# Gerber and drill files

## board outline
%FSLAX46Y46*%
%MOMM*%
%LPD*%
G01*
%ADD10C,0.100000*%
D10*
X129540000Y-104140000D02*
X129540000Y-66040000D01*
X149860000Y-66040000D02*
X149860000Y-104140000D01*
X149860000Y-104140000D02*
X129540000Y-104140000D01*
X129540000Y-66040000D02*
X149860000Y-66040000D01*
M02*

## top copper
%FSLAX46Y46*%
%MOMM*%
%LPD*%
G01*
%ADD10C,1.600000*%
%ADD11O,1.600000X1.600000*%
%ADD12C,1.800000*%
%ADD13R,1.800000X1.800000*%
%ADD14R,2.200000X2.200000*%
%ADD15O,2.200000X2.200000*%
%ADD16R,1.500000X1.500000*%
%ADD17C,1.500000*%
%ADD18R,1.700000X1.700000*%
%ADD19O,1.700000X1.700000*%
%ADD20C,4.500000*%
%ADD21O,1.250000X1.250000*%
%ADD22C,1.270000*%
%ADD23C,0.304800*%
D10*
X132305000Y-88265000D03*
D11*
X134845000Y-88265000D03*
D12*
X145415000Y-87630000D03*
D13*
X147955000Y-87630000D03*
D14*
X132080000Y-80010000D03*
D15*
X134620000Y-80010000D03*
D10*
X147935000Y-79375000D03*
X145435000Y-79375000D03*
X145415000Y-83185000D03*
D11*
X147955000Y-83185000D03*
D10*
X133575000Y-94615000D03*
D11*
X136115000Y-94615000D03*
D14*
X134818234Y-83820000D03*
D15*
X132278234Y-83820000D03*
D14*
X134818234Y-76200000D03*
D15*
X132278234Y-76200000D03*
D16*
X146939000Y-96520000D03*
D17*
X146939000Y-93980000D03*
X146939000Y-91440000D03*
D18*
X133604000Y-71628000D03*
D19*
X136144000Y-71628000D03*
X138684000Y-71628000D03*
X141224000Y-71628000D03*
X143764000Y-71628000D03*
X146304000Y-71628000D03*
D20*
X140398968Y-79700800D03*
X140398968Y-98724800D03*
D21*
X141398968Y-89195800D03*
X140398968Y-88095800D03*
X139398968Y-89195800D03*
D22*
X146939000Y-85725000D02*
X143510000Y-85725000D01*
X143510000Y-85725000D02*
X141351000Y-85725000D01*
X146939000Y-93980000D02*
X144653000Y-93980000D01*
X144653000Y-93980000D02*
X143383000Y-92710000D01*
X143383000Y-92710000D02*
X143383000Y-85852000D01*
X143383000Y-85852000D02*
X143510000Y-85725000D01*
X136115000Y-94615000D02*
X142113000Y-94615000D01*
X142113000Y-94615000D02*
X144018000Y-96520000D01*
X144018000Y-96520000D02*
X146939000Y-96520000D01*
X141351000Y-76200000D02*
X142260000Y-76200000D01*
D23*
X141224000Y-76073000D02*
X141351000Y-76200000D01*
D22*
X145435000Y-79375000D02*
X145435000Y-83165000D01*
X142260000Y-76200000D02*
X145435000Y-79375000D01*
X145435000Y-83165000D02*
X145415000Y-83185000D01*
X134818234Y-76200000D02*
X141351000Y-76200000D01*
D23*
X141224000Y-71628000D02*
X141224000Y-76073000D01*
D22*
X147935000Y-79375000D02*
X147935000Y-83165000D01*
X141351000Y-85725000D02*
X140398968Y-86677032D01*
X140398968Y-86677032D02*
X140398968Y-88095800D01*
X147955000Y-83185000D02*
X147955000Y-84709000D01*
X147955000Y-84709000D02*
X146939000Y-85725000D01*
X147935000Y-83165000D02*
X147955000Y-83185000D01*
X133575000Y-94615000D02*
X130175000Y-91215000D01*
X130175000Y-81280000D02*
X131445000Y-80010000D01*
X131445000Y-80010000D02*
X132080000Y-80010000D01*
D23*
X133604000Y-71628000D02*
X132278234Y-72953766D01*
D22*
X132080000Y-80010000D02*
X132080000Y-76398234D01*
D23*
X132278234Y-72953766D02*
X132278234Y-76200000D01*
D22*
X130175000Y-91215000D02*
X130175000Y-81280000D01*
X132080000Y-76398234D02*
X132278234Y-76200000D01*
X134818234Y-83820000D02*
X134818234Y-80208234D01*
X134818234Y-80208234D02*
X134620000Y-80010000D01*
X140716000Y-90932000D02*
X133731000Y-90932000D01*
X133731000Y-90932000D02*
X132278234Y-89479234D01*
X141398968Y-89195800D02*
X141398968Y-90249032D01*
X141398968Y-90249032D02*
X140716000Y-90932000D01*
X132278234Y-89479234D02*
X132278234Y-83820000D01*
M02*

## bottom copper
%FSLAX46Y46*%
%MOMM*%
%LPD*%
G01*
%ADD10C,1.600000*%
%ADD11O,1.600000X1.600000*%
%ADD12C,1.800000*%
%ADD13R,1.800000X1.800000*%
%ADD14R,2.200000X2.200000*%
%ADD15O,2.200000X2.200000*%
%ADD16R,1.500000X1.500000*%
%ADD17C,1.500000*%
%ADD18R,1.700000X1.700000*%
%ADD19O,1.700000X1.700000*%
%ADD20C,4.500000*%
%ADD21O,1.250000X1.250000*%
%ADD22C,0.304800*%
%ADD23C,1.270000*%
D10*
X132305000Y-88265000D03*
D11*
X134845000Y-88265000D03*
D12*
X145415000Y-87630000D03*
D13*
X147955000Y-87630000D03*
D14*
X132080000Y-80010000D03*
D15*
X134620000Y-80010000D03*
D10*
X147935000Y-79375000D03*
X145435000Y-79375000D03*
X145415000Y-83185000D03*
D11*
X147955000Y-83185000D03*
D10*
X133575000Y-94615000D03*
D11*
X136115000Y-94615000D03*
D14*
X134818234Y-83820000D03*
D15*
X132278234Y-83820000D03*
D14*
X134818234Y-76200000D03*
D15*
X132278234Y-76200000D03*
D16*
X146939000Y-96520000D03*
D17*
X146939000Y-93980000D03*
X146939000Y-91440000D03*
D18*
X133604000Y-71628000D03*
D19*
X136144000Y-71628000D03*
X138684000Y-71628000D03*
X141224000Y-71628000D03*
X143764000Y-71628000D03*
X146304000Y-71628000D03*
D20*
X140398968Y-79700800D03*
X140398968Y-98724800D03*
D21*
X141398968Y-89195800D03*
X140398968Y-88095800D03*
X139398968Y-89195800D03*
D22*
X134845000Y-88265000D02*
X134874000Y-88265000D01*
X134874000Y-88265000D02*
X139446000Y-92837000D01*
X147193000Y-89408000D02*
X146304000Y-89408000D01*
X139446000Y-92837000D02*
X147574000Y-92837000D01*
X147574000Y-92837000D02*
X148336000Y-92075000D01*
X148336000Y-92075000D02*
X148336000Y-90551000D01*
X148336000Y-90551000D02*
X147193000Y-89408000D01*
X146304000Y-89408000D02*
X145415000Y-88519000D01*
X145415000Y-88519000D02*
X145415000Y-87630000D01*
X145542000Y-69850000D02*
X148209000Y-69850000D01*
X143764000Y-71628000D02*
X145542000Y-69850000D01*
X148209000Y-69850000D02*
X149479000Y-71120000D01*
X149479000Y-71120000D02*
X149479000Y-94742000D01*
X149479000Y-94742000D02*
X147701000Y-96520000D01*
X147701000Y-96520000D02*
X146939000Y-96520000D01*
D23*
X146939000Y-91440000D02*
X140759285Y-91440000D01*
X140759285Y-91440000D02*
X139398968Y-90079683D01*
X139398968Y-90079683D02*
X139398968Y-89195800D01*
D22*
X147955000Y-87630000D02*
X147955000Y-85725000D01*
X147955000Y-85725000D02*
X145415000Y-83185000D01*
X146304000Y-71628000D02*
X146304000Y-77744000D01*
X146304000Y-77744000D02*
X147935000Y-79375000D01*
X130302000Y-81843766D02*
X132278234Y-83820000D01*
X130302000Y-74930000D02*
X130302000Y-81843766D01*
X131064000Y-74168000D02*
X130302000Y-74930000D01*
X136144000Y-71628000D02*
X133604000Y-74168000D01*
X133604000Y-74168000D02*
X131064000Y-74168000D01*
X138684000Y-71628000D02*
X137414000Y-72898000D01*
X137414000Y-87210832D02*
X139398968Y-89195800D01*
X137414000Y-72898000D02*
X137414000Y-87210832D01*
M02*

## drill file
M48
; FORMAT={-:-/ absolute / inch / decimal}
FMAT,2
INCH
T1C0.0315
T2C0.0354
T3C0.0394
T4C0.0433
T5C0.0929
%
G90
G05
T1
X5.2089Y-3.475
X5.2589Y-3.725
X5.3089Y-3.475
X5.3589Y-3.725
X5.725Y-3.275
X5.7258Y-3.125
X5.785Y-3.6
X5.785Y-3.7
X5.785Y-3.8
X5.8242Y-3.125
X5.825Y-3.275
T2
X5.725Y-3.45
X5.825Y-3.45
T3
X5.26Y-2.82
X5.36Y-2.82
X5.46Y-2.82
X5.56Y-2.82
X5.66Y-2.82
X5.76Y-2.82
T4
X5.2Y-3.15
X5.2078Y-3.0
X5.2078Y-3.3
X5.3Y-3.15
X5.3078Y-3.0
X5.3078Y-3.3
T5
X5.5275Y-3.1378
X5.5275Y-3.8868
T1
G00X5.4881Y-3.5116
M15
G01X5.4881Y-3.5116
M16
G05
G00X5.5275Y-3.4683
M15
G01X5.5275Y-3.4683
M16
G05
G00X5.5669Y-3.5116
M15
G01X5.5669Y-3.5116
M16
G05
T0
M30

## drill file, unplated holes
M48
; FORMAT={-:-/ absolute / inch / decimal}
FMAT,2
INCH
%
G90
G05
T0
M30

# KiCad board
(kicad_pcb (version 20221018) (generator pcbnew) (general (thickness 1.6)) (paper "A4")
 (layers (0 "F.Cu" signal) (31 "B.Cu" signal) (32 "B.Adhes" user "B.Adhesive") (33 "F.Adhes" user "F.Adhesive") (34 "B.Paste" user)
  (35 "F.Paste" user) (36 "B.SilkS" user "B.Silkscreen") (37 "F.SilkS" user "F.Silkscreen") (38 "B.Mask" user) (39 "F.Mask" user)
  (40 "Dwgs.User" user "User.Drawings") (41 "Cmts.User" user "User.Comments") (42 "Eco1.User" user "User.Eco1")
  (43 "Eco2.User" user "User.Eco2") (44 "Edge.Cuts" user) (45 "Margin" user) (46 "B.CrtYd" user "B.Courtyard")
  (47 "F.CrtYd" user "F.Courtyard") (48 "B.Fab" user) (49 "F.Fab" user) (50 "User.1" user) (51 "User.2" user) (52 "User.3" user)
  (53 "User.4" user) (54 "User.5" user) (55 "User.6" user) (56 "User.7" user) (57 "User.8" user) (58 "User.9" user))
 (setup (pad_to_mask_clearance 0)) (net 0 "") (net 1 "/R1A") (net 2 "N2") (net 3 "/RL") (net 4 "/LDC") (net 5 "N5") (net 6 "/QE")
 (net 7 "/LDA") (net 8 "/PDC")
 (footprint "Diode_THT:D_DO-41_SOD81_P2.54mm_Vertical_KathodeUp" (layer "F.Cu") (at 132.08 80.01)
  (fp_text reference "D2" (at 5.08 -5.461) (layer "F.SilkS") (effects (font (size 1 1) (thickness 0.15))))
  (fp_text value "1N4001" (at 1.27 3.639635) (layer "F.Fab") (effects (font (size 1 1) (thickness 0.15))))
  (pad "1" thru_hole rect (at 0 0) (size 2.2 2.2) (drill 1.1) (layers "*.Cu" "*.Mask") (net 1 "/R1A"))
  (pad "2" thru_hole oval (at 2.54 0) (size 2.2 2.2) (drill 1.1) (layers "*.Cu" "*.Mask") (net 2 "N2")))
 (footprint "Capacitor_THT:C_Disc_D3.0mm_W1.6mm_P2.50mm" (layer "F.Cu") (at 145.435 79.375)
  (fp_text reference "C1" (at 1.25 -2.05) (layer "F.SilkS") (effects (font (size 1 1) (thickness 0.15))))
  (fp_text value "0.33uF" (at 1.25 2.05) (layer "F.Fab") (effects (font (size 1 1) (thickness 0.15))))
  (pad "1" thru_hole circle (at 0 0) (size 1.6 1.6) (drill 0.8) (layers "*.Cu" "*.Mask") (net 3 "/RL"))
  (pad "2" thru_hole circle (at 2.5 0) (size 1.6 1.6) (drill 0.8) (layers "*.Cu" "*.Mask") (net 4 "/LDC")))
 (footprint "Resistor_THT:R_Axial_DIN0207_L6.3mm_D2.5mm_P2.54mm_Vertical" (layer "F.Cu") (at 145.415 83.185)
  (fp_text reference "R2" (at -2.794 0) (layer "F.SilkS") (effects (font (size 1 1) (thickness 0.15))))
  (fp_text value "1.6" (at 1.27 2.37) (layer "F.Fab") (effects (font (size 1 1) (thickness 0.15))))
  (pad "1" thru_hole circle (at 0 0) (size 1.6 1.6) (drill 0.8) (layers "*.Cu" "*.Mask") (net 3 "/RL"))
  (pad "2" thru_hole oval (at 2.54 0) (size 1.6 1.6) (drill 0.8) (layers "*.Cu" "*.Mask") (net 4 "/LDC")))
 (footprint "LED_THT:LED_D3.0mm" (layer "F.Cu") (at 147.955 87.63 180)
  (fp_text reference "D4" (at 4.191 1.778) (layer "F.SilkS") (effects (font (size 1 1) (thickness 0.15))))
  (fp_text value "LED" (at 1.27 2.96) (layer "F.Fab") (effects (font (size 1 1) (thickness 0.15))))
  (pad "1" thru_hole rect (at 0 0 180) (size 1.8 1.8) (drill 0.9) (layers "*.Cu" "*.Mask") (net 3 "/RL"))
  (pad "2" thru_hole circle (at 2.54 0 180) (size 1.8 1.8) (drill 0.9) (layers "*.Cu" "*.Mask") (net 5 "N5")))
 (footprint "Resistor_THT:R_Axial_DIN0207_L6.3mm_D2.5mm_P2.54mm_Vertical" (layer "F.Cu") (at 133.575 94.615)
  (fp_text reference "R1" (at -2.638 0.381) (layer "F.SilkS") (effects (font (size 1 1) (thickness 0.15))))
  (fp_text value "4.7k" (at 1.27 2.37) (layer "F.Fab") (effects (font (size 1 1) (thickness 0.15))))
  (pad "1" thru_hole circle (at 0 0) (size 1.6 1.6) (drill 0.8) (layers "*.Cu" "*.Mask") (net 1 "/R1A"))
  (pad "2" thru_hole oval (at 2.54 0) (size 1.6 1.6) (drill 0.8) (layers "*.Cu" "*.Mask") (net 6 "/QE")))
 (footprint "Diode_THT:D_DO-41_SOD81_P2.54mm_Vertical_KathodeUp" (layer "F.Cu") (at 134.818234 83.82 180)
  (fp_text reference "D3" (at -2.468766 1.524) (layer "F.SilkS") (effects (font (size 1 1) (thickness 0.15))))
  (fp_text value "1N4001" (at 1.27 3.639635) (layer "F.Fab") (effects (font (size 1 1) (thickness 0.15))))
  (pad "1" thru_hole rect (at 0 0 180) (size 2.2 2.2) (drill 1.1) (layers "*.Cu" "*.Mask") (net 2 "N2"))
  (pad "2" thru_hole oval (at 2.54 0 180) (size 2.2 2.2) (drill 1.1) (layers "*.Cu" "*.Mask") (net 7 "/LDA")))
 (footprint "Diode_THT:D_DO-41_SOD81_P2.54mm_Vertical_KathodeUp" (layer "F.Cu") (at 134.818234 76.2 180)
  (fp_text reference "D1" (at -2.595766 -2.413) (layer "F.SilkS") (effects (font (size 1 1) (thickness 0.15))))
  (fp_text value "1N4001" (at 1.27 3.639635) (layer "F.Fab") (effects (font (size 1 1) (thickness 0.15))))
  (pad "1" thru_hole rect (at 0 0 180) (size 2.2 2.2) (drill 1.1) (layers "*.Cu" "*.Mask") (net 3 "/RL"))
  (pad "2" thru_hole oval (at 2.54 0 180) (size 2.2 2.2) (drill 1.1) (layers "*.Cu" "*.Mask") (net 1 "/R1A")))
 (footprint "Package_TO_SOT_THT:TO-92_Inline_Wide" (layer "F.Cu") (at 146.939 96.52 90)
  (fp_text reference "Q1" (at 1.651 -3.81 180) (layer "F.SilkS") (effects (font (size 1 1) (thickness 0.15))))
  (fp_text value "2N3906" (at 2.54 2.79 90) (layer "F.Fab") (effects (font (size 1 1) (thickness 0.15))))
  (pad "1" thru_hole rect (at 0 0 90) (size 1.5 1.5) (drill 0.8) (layers "*.Cu" "*.Mask") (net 6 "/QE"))
  (pad "2" thru_hole circle (at 2.54 0 90) (size 1.5 1.5) (drill 0.8) (layers "*.Cu" "*.Mask") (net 4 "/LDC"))
  (pad "3" thru_hole circle (at 5.08 0 90) (size 1.5 1.5) (drill 0.8) (layers "*.Cu" "*.Mask") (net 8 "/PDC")))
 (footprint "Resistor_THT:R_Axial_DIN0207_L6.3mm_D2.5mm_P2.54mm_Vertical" (layer "F.Cu") (at 132.305 88.265)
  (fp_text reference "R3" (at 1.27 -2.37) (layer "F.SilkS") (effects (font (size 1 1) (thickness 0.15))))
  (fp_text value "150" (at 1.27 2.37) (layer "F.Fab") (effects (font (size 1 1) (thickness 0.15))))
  (pad "1" thru_hole circle (at 0 0) (size 1.6 1.6) (drill 0.8) (layers "*.Cu" "*.Mask") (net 7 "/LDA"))
  (pad "2" thru_hole oval (at 2.54 0) (size 1.6 1.6) (drill 0.8) (layers "*.Cu" "*.Mask") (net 5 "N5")))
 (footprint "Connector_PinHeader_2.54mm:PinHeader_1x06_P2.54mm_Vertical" (layer "F.Cu") (at 133.604 71.628 90)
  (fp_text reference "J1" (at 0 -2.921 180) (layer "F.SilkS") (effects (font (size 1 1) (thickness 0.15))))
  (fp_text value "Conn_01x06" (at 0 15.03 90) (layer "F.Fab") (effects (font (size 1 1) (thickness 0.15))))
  (pad "1" thru_hole rect (at 0 0 90) (size 1.7 1.7) (drill 1) (layers "*.Cu" "*.Mask") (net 1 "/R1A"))
  (pad "2" thru_hole oval (at 0 2.54 90) (size 1.7 1.7) (drill 1) (layers "*.Cu" "*.Mask") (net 7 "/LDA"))
  (pad "3" thru_hole oval (at 0 5.08 90) (size 1.7 1.7) (drill 1) (layers "*.Cu" "*.Mask") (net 8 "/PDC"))
  (pad "4" thru_hole oval (at 0 7.62 90) (size 1.7 1.7) (drill 1) (layers "*.Cu" "*.Mask") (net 3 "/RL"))
  (pad "5" thru_hole oval (at 0 10.16 90) (size 1.7 1.7) (drill 1) (layers "*.Cu" "*.Mask") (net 6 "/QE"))
  (pad "6" thru_hole oval (at 0 12.7 90) (size 1.7 1.7) (drill 1) (layers "*.Cu" "*.Mask") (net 4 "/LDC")))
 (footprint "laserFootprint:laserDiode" (layer "B.Cu") (at 141.398968 89.1958 90)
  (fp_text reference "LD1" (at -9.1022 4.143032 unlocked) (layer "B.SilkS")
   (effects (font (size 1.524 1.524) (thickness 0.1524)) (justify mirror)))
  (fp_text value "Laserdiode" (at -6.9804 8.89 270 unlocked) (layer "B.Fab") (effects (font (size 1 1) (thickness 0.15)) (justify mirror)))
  (pad "1" thru_hole oval (at 0 -2) (size 1.25 1.25) (drill oval 0.8) (layers "*.Cu" "*.Mask") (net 8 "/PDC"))
  (pad "2" thru_hole oval (at 1.1 -1) (size 1.25 1.25) (drill oval 0.8) (layers "*.Cu" "*.Mask") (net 4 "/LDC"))
  (pad "3" thru_hole oval (at 0 0) (size 1.25 1.25) (drill oval 0.8) (layers "*.Cu" "*.Mask") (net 7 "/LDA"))
  (pad "4" thru_hole circle (at -9.529 -1 90) (size 4.5 4.5) (drill 2.36) (layers "*.Cu" "*.Mask"))
  (pad "4" thru_hole circle (at 9.495 -1 90) (size 4.5 4.5) (drill 2.36) (layers "*.Cu" "*.Mask")))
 (gr_line (start 129.54 104.14) (end 129.54 66.04) (stroke (width 0.1) (type default)) (layer "Edge.Cuts"))
 (gr_line (start 149.86 66.04) (end 149.86 104.14) (stroke (width 0.1) (type default)) (layer "Edge.Cuts"))
 (gr_line (start 149.86 104.14) (end 129.54 104.14) (stroke (width 0.1) (type default)) (layer "Edge.Cuts"))
 (gr_line (start 129.54 66.04) (end 149.86 66.04) (stroke (width 0.1) (type default)) (layer "Edge.Cuts"))
 (segment (start 141.351 76.2) (end 142.26 76.2) (width 1.27) (layer "F.Cu") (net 3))
 (segment (start 141.224 76.073) (end 141.351 76.2) (width 0.3048) (layer "F.Cu") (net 3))
 (segment (start 145.435 79.375) (end 145.435 83.165) (width 1.27) (layer "F.Cu") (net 3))
 (segment (start 142.26 76.2) (end 145.435 79.375) (width 1.27) (layer "F.Cu") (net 3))
 (segment (start 145.435 83.165) (end 145.415 83.185) (width 1.27) (layer "F.Cu") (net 3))
 (segment (start 134.818234 76.2) (end 141.351 76.2) (width 1.27) (layer "F.Cu") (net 3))
 (segment (start 141.224 71.628) (end 141.224 76.073) (width 0.3048) (layer "F.Cu") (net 3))
 (segment (start 147.955 87.63) (end 147.955 85.725) (width 0.3048) (layer "B.Cu") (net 3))
 (segment (start 147.955 85.725) (end 145.415 83.185) (width 0.3048) (layer "B.Cu") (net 3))
 (segment (start 147.935 79.375) (end 147.935 83.165) (width 1.27) (layer "F.Cu") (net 4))
 (segment (start 141.351 85.725) (end 140.398968 86.677032) (width 1.27) (layer "F.Cu") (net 4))
 (segment (start 143.51 85.725) (end 141.351 85.725) (width 1.27) (layer "F.Cu") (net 4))
 (segment (start 146.939 93.98) (end 144.653 93.98) (width 1.27) (layer "F.Cu") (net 4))
 (segment (start 143.383 85.852) (end 143.51 85.725) (width 1.27) (layer "F.Cu") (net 4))
 (segment (start 140.398968 86.677032) (end 140.398968 88.0958) (width 1.27) (layer "F.Cu") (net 4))
 (segment (start 143.383 92.71) (end 143.383 85.852) (width 1.27) (layer "F.Cu") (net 4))
 (segment (start 147.955 83.185) (end 147.955 84.709) (width 1.27) (layer "F.Cu") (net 4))
 (segment (start 144.653 93.98) (end 143.383 92.71) (width 1.27) (layer "F.Cu") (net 4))
 (segment (start 147.955 84.709) (end 146.939 85.725) (width 1.27) (layer "F.Cu") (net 4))
 (segment (start 146.939 85.725) (end 143.51 85.725) (width 1.27) (layer "F.Cu") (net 4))
 (segment (start 147.935 83.165) (end 147.955 83.185) (width 1.27) (layer "F.Cu") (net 4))
 (segment (start 146.304 71.628) (end 146.304 77.744) (width 0.3048) (layer "B.Cu") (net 4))
 (segment (start 146.304 77.744) (end 147.935 79.375) (width 0.3048) (layer "B.Cu") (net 4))
 (segment (start 133.575 94.615) (end 130.175 91.215) (width 1.27) (layer "F.Cu") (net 1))
 (segment (start 130.175 81.28) (end 131.445 80.01) (width 1.27) (layer "F.Cu") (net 1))
 (segment (start 131.445 80.01) (end 132.08 80.01) (width 1.27) (layer "F.Cu") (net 1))
 (segment (start 133.604 71.628) (end 132.278234 72.953766) (width 0.3048) (layer "F.Cu") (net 1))
 (segment (start 132.08 80.01) (end 132.08 76.398234) (width 1.27) (layer "F.Cu") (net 1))
 (segment (start 132.278234 72.953766) (end 132.278234 76.2) (width 0.3048) (layer "F.Cu") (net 1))
 (segment (start 130.175 91.215) (end 130.175 81.28) (width 1.27) (layer "F.Cu") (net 1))
 (segment (start 132.08 76.398234) (end 132.278234 76.2) (width 1.27) (layer "F.Cu") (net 1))
 (segment (start 134.818234 83.82) (end 134.818234 80.208234) (width 1.27) (layer "F.Cu") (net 2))
 (segment (start 134.818234 80.208234) (end 134.62 80.01) (width 1.27) (layer "F.Cu") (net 2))
 (segment (start 140.716 90.932) (end 133.731 90.932) (width 1.27) (layer "F.Cu") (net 7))
 (segment (start 133.731 90.932) (end 132.278234 89.479234) (width 1.27) (layer "F.Cu") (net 7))
 (segment (start 141.398968 89.1958) (end 141.398968 90.249032) (width 1.27) (layer "F.Cu") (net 7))
 (segment (start 141.398968 90.249032) (end 140.716 90.932) (width 1.27) (layer "F.Cu") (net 7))
 (segment (start 132.278234 89.479234) (end 132.278234 83.82) (width 1.27) (layer "F.Cu") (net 7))
 (segment (start 130.302 81.843766) (end 132.278234 83.82) (width 0.3048) (layer "B.Cu") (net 7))
 (segment (start 130.302 74.93) (end 130.302 81.843766) (width 0.3048) (layer "B.Cu") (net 7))
 (segment (start 131.064 74.168) (end 130.302 74.93) (width 0.3048) (layer "B.Cu") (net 7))
 (segment (start 136.144 71.628) (end 133.604 74.168) (width 0.3048) (layer "B.Cu") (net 7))
 (segment (start 133.604 74.168) (end 131.064 74.168) (width 0.3048) (layer "B.Cu") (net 7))
 (segment (start 138.684 71.628) (end 137.414 72.898) (width 0.3048) (layer "B.Cu") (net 8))
 (segment (start 139.398968 90.079683) (end 139.398968 89.1958) (width 1.27) (layer "B.Cu") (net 8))
 (segment (start 137.414 87.210832) (end 139.398968 89.1958) (width 0.3048) (layer "B.Cu") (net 8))
 (segment (start 137.414 72.898) (end 137.414 87.210832) (width 0.3048) (layer "B.Cu") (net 8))
 (segment (start 140.759285 91.44) (end 139.398968 90.079683) (width 1.27) (layer "B.Cu") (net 8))
 (segment (start 146.939 91.44) (end 140.759285 91.44) (width 1.27) (layer "B.Cu") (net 8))
 (segment (start 142.113 94.615) (end 144.018 96.52) (width 1.27) (layer "F.Cu") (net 6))
 (segment (start 136.115 94.615) (end 142.113 94.615) (width 1.27) (layer "F.Cu") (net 6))
 (segment (start 144.018 96.52) (end 146.939 96.52) (width 1.27) (layer "F.Cu") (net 6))
 (segment (start 149.479 71.12) (end 149.479 94.742) (width 0.3048) (layer "B.Cu") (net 6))
 (segment (start 145.542 69.85) (end 148.209 69.85) (width 0.3048) (layer "B.Cu") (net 6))
 (segment (start 149.479 94.742) (end 147.701 96.52) (width 0.3048) (layer "B.Cu") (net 6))
 (segment (start 147.701 96.52) (end 146.939 96.52) (width 0.3048) (layer "B.Cu") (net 6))
 (segment (start 148.209 69.85) (end 149.479 71.12) (width 0.3048) (layer "B.Cu") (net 6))
 (segment (start 143.764 71.628) (end 145.542 69.85) (width 0.3048) (layer "B.Cu") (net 6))
 (segment (start 148.336 92.075) (end 148.336 90.551) (width 0.3048) (layer "B.Cu") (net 5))
 (segment (start 147.193 89.408) (end 146.304 89.408) (width 0.3048) (layer "B.Cu") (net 5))
 (segment (start 147.574 92.837) (end 148.336 92.075) (width 0.3048) (layer "B.Cu") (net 5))
 (segment (start 134.845 88.265) (end 134.874 88.265) (width 0.3048) (layer "B.Cu") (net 5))
 (segment (start 146.304 89.408) (end 145.415 88.519) (width 0.3048) (layer "B.Cu") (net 5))
 (segment (start 145.415 88.519) (end 145.415 87.63) (width 0.3048) (layer "B.Cu") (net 5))
 (segment (start 139.446 92.837) (end 147.574 92.837) (width 0.3048) (layer "B.Cu") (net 5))
 (segment (start 134.874 88.265) (end 139.446 92.837) (width 0.3048) (layer "B.Cu") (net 5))
 (segment (start 148.336 90.551) (end 147.193 89.408) (width 0.3048) (layer "B.Cu") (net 5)))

